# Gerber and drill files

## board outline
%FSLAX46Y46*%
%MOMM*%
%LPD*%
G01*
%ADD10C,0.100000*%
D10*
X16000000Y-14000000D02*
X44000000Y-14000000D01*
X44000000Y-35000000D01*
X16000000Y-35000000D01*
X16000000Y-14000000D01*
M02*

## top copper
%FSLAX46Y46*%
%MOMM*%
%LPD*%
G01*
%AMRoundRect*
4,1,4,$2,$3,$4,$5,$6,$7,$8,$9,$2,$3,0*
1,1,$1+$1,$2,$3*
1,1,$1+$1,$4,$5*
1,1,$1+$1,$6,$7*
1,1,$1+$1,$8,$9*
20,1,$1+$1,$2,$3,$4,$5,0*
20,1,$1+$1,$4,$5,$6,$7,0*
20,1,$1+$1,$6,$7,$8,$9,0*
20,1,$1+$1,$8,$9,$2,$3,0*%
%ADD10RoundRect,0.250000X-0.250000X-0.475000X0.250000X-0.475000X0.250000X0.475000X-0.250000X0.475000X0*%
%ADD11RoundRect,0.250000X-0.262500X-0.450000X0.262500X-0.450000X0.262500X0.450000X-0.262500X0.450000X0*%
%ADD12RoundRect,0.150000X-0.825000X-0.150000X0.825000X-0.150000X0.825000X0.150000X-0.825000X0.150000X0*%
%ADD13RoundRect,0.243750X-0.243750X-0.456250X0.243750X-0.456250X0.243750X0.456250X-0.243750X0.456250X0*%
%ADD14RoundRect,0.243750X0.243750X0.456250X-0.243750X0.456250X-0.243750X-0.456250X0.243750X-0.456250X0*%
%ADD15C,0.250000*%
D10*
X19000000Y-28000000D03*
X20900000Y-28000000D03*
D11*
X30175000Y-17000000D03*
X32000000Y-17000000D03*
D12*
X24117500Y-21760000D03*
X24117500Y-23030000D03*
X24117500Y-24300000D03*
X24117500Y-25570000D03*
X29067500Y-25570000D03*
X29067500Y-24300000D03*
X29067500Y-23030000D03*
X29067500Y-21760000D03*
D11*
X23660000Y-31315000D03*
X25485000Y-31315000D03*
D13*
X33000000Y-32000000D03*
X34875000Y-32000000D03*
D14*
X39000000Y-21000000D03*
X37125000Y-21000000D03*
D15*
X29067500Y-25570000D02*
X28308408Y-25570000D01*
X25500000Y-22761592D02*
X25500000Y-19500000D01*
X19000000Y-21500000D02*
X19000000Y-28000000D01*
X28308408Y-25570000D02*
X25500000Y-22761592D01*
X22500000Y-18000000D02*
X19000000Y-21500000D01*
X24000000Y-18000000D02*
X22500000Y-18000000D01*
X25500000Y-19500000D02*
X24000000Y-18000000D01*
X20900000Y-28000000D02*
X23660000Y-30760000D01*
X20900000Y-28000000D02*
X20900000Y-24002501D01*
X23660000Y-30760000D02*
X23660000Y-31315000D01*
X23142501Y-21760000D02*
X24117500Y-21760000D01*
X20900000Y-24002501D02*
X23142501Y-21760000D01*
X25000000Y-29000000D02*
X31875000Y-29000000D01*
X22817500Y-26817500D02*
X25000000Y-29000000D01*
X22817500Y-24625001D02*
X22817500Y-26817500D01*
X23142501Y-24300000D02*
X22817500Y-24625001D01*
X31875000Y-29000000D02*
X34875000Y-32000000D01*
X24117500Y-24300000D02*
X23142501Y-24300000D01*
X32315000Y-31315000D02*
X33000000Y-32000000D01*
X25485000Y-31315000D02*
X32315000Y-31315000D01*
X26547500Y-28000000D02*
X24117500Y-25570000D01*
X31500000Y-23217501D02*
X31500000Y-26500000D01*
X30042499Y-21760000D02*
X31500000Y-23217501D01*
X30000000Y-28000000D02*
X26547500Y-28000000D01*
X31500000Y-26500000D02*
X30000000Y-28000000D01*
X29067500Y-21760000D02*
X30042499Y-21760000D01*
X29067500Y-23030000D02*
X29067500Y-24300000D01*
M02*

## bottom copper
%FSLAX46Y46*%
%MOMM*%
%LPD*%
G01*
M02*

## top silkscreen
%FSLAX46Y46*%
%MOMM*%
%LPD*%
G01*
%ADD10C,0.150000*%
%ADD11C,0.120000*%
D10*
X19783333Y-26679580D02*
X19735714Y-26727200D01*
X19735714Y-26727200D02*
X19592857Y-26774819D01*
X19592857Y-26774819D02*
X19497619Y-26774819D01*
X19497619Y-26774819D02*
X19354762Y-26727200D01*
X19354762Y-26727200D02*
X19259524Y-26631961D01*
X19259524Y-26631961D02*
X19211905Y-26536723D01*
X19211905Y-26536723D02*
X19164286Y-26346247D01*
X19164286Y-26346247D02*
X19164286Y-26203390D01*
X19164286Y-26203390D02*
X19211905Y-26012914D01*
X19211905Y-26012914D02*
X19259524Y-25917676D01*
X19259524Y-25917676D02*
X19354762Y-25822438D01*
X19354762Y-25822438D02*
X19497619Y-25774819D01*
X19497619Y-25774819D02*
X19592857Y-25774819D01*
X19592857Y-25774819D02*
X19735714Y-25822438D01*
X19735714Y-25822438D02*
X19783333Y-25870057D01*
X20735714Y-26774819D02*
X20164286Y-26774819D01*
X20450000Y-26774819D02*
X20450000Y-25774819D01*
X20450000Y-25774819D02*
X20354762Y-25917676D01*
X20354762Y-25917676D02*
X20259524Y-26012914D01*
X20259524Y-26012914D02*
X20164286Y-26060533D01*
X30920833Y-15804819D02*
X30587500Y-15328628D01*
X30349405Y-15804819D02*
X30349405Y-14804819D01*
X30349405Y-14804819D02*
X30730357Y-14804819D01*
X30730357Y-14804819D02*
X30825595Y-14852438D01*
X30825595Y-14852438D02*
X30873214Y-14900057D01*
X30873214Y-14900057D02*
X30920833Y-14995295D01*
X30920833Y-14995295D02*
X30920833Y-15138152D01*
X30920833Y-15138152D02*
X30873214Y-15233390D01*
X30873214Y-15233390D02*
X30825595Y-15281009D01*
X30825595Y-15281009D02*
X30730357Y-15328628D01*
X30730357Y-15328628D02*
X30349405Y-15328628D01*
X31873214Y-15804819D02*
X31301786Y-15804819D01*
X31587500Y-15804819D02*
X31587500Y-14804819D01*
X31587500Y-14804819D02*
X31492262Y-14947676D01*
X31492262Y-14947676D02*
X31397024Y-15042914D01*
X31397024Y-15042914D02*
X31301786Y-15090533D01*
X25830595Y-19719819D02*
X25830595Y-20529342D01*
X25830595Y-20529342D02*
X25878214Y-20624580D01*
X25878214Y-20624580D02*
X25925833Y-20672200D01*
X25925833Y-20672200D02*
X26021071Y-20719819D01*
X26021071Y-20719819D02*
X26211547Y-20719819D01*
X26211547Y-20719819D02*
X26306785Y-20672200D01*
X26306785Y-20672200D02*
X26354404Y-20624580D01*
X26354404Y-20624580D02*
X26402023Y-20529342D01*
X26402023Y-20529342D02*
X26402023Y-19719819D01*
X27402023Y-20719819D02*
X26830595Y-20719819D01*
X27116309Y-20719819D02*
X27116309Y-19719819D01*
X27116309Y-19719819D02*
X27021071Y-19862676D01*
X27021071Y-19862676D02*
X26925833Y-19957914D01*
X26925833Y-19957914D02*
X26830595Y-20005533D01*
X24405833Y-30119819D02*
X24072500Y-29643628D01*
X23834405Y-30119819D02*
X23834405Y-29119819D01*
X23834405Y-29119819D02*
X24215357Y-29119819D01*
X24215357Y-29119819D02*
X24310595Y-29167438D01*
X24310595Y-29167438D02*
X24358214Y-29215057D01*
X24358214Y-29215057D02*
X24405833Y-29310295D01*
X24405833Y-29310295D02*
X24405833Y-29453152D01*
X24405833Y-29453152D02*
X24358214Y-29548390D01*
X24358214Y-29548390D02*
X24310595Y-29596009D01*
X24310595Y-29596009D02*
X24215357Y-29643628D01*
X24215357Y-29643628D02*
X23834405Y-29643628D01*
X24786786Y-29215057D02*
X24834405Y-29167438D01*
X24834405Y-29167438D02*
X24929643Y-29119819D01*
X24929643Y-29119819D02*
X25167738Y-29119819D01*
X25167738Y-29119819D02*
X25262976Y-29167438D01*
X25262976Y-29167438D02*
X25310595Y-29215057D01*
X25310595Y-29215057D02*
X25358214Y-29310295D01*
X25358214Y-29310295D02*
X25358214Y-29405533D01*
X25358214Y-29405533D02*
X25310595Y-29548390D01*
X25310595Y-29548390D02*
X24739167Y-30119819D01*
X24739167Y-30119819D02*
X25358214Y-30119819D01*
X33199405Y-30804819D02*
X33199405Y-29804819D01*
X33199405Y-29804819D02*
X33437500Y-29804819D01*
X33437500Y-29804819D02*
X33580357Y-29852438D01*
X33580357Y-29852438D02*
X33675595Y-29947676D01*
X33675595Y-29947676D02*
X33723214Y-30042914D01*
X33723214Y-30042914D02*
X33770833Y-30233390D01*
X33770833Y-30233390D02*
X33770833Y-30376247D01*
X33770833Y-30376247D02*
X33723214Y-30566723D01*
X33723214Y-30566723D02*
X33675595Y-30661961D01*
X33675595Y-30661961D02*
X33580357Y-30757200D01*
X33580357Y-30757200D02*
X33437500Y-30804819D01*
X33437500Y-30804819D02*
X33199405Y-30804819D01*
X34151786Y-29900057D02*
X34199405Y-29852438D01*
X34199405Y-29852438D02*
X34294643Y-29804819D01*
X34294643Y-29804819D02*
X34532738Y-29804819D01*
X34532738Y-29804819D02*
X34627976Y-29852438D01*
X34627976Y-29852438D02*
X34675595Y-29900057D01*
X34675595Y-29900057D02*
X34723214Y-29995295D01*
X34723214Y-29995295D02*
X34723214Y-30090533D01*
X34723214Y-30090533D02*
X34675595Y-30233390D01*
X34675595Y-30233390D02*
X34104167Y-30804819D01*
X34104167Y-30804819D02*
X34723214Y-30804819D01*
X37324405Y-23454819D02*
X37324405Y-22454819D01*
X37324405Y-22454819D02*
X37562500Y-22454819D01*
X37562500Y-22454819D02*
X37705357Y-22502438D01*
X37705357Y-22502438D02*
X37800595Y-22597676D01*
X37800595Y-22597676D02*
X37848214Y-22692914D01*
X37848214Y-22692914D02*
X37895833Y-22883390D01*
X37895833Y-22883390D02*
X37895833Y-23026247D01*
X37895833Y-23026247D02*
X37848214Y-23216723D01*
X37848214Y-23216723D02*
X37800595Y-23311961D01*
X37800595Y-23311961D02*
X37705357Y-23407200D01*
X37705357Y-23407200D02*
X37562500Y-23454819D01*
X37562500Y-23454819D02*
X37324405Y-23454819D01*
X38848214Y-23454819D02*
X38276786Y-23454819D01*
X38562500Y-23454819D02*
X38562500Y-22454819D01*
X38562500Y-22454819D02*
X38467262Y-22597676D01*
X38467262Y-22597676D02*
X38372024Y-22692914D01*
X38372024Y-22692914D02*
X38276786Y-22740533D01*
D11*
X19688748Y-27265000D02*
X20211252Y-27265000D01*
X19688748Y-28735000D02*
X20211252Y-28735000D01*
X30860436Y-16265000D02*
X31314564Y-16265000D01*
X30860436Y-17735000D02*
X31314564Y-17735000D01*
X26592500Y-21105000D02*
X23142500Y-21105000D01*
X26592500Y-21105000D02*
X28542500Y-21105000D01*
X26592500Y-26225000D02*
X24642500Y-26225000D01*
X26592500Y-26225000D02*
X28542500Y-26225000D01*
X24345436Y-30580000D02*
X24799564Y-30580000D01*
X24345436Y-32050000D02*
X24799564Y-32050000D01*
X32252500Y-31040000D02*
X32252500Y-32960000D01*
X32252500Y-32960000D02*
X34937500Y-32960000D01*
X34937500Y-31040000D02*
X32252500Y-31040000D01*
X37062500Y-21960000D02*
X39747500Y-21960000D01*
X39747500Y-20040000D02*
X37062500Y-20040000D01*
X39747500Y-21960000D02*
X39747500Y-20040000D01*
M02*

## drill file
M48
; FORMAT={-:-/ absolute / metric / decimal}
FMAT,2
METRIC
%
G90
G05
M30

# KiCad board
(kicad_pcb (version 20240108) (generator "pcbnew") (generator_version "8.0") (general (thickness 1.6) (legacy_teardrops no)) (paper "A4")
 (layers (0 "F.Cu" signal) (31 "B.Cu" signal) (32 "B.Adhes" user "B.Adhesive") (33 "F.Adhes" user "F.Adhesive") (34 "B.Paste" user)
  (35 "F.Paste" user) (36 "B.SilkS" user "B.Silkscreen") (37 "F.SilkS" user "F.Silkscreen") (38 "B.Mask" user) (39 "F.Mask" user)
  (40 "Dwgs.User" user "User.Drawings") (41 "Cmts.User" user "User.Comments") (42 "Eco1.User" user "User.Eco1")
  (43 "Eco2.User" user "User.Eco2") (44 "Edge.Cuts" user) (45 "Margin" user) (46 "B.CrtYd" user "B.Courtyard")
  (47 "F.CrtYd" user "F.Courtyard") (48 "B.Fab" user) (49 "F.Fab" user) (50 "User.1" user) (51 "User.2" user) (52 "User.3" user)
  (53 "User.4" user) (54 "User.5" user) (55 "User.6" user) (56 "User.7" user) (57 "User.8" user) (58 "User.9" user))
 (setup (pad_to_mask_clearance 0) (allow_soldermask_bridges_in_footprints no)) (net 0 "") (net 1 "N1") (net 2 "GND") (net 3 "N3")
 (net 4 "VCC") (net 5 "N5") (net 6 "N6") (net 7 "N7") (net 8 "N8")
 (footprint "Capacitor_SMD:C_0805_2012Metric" (layer "F.Cu") (at 19.95 28)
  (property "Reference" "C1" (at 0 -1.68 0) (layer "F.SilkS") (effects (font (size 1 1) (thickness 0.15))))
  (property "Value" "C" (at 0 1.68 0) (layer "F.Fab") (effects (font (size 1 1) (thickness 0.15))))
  (fp_line (start -0.261252 -0.735) (end 0.261252 -0.735) (stroke (width 0.12) (type solid)) (layer "F.SilkS"))
  (fp_line (start -0.261252 0.735) (end 0.261252 0.735) (stroke (width 0.12) (type solid)) (layer "F.SilkS"))
  (pad "1" smd roundrect (at -0.95 0) (size 1 1.45) (layers "F.Cu" "F.Paste" "F.Mask") (roundrect_rratio 0.25) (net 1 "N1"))
  (pad "2" smd roundrect (at 0.95 0) (size 1 1.45) (layers "F.Cu" "F.Paste" "F.Mask") (roundrect_rratio 0.25) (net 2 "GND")))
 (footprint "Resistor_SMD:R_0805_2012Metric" (layer "F.Cu") (at 31.0875 17)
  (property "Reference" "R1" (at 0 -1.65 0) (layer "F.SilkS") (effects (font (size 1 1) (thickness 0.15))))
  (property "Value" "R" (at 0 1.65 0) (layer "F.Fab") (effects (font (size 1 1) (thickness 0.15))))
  (fp_line (start -0.227064 -0.735) (end 0.227064 -0.735) (stroke (width 0.12) (type solid)) (layer "F.SilkS"))
  (fp_line (start -0.227064 0.735) (end 0.227064 0.735) (stroke (width 0.12) (type solid)) (layer "F.SilkS"))
  (pad "1" smd roundrect (at -0.9125 0) (size 1.025 1.4) (layers "F.Cu" "F.Paste" "F.Mask") (roundrect_rratio 0.243902) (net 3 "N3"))
  (pad "2" smd roundrect (at 0.9125 0) (size 1.025 1.4) (layers "F.Cu" "F.Paste" "F.Mask") (roundrect_rratio 0.243902) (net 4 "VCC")))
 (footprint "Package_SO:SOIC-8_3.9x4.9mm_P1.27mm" (layer "F.Cu") (at 26.5925 23.665)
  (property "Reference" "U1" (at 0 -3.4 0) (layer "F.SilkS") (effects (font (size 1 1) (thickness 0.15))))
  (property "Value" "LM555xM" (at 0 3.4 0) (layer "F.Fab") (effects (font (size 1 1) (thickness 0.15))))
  (fp_line (start 0 -2.56) (end -3.45 -2.56) (stroke (width 0.12) (type solid)) (layer "F.SilkS"))
  (fp_line (start 0 -2.56) (end 1.95 -2.56) (stroke (width 0.12) (type solid)) (layer "F.SilkS"))
  (fp_line (start 0 2.56) (end -1.95 2.56) (stroke (width 0.12) (type solid)) (layer "F.SilkS"))
  (fp_line (start 0 2.56) (end 1.95 2.56) (stroke (width 0.12) (type solid)) (layer "F.SilkS"))
  (pad "1" smd roundrect (at -2.475 -1.905) (size 1.95 0.6) (layers "F.Cu" "F.Paste" "F.Mask") (roundrect_rratio 0.25) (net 2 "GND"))
  (pad "2" smd roundrect (at -2.475 -0.635) (size 1.95 0.6) (layers "F.Cu" "F.Paste" "F.Mask") (roundrect_rratio 0.25) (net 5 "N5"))
  (pad "3" smd roundrect (at -2.475 0.635) (size 1.95 0.6) (layers "F.Cu" "F.Paste" "F.Mask") (roundrect_rratio 0.25) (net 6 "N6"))
  (pad "4" smd roundrect (at -2.475 1.905) (size 1.95 0.6) (layers "F.Cu" "F.Paste" "F.Mask") (roundrect_rratio 0.25) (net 4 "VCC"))
  (pad "5" smd roundrect (at 2.475 1.905) (size 1.95 0.6) (layers "F.Cu" "F.Paste" "F.Mask") (roundrect_rratio 0.25) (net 1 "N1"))
  (pad "6" smd roundrect (at 2.475 0.635) (size 1.95 0.6) (layers "F.Cu" "F.Paste" "F.Mask") (roundrect_rratio 0.25) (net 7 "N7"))
  (pad "7" smd roundrect (at 2.475 -0.635) (size 1.95 0.6) (layers "F.Cu" "F.Paste" "F.Mask") (roundrect_rratio 0.25) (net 7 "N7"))
  (pad "8" smd roundrect (at 2.475 -1.905) (size 1.95 0.6) (layers "F.Cu" "F.Paste" "F.Mask") (roundrect_rratio 0.25) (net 4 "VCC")))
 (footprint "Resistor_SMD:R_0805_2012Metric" (layer "F.Cu") (at 24.5725 31.315)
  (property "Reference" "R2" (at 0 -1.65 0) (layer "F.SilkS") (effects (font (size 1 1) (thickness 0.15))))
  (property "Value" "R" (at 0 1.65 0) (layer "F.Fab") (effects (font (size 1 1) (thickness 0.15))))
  (fp_line (start -0.227064 -0.735) (end 0.227064 -0.735) (stroke (width 0.12) (type solid)) (layer "F.SilkS"))
  (fp_line (start -0.227064 0.735) (end 0.227064 0.735) (stroke (width 0.12) (type solid)) (layer "F.SilkS"))
  (pad "1" smd roundrect (at -0.9125 0) (size 1.025 1.4) (layers "F.Cu" "F.Paste" "F.Mask") (roundrect_rratio 0.243902) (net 2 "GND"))
  (pad "2" smd roundrect (at 0.9125 0) (size 1.025 1.4) (layers "F.Cu" "F.Paste" "F.Mask") (roundrect_rratio 0.243902) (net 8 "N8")))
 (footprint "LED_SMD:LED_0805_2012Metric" (layer "F.Cu") (at 33.9375 32)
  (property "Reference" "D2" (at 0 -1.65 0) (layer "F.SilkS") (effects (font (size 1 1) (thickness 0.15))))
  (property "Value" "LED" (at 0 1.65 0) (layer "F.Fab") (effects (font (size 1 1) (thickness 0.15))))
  (fp_line (start -1.685 -0.96) (end -1.685 0.96) (stroke (width 0.12) (type solid)) (layer "F.SilkS"))
  (fp_line (start -1.685 0.96) (end 1 0.96) (stroke (width 0.12) (type solid)) (layer "F.SilkS"))
  (fp_line (start 1 -0.96) (end -1.685 -0.96) (stroke (width 0.12) (type solid)) (layer "F.SilkS"))
  (pad "1" smd roundrect (at -0.9375 0) (size 0.975 1.4) (layers "F.Cu" "F.Paste" "F.Mask") (roundrect_rratio 0.25) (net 8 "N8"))
  (pad "2" smd roundrect (at 0.9375 0) (size 0.975 1.4) (layers "F.Cu" "F.Paste" "F.Mask") (roundrect_rratio 0.25) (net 6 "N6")))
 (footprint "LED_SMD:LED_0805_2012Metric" (layer "F.Cu") (at 38.0625 21 180)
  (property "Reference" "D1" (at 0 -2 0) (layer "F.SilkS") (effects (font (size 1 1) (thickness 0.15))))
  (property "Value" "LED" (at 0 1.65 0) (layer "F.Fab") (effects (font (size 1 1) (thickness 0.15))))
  (fp_line (start 1 -0.96) (end -1.685 -0.96) (stroke (width 0.12) (type solid)) (layer "F.SilkS"))
  (fp_line (start -1.685 0.96) (end 1 0.96) (stroke (width 0.12) (type solid)) (layer "F.SilkS"))
  (fp_line (start -1.685 -0.96) (end -1.685 0.96) (stroke (width 0.12) (type solid)) (layer "F.SilkS"))
  (pad "1" smd roundrect (at -0.9375 0 180) (size 0.975 1.4) (layers "F.Cu" "F.Paste" "F.Mask") (roundrect_rratio 0.25) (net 6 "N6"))
  (pad "2" smd roundrect (at 0.9375 0 180) (size 0.975 1.4) (layers "F.Cu" "F.Paste" "F.Mask") (roundrect_rratio 0.25) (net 3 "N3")))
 (gr_rect (start 16 14) (end 44 35) (stroke (width 0.1) (type default)) (fill none) (layer "Edge.Cuts"))
 (segment (start 29.0675 25.57) (end 28.308408 25.57) (width 0.25) (layer "F.Cu") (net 1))
 (segment (start 25.5 22.761592) (end 25.5 19.5) (width 0.25) (layer "F.Cu") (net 1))
 (segment (start 19 21.5) (end 19 28) (width 0.25) (layer "F.Cu") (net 1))
 (segment (start 28.308408 25.57) (end 25.5 22.761592) (width 0.25) (layer "F.Cu") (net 1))
 (segment (start 22.5 18) (end 19 21.5) (width 0.25) (layer "F.Cu") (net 1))
 (segment (start 24 18) (end 22.5 18) (width 0.25) (layer "F.Cu") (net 1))
 (segment (start 25.5 19.5) (end 24 18) (width 0.25) (layer "F.Cu") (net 1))
 (segment (start 20.9 28) (end 23.66 30.76) (width 0.25) (layer "F.Cu") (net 2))
 (segment (start 20.9 28) (end 20.9 24.002501) (width 0.25) (layer "F.Cu") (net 2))
 (segment (start 23.66 30.76) (end 23.66 31.315) (width 0.25) (layer "F.Cu") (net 2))
 (segment (start 23.142501 21.76) (end 24.1175 21.76) (width 0.25) (layer "F.Cu") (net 2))
 (segment (start 20.9 24.002501) (end 23.142501 21.76) (width 0.25) (layer "F.Cu") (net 2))
 (segment (start 25 29) (end 31.875 29) (width 0.25) (layer "F.Cu") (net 6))
 (segment (start 22.8175 26.8175) (end 25 29) (width 0.25) (layer "F.Cu") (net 6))
 (segment (start 22.8175 24.625001) (end 22.8175 26.8175) (width 0.25) (layer "F.Cu") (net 6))
 (segment (start 23.142501 24.3) (end 22.8175 24.625001) (width 0.25) (layer "F.Cu") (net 6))
 (segment (start 31.875 29) (end 34.875 32) (width 0.25) (layer "F.Cu") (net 6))
 (segment (start 24.1175 24.3) (end 23.142501 24.3) (width 0.25) (layer "F.Cu") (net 6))
 (segment (start 32.315 31.315) (end 33 32) (width 0.25) (layer "F.Cu") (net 8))
 (segment (start 25.485 31.315) (end 32.315 31.315) (width 0.25) (layer "F.Cu") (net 8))
 (segment (start 26.5475 28) (end 24.1175 25.57) (width 0.25) (layer "F.Cu") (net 4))
 (segment (start 31.5 23.217501) (end 31.5 26.5) (width 0.25) (layer "F.Cu") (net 4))
 (segment (start 30.042499 21.76) (end 31.5 23.217501) (width 0.25) (layer "F.Cu") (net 4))
 (segment (start 30 28) (end 26.5475 28) (width 0.25) (layer "F.Cu") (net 4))
 (segment (start 31.5 26.5) (end 30 28) (width 0.25) (layer "F.Cu") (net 4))
 (segment (start 29.0675 21.76) (end 30.042499 21.76) (width 0.25) (layer "F.Cu") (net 4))
 (segment (start 29.0675 23.03) (end 29.0675 24.3) (width 0.25) (layer "F.Cu") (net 7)))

